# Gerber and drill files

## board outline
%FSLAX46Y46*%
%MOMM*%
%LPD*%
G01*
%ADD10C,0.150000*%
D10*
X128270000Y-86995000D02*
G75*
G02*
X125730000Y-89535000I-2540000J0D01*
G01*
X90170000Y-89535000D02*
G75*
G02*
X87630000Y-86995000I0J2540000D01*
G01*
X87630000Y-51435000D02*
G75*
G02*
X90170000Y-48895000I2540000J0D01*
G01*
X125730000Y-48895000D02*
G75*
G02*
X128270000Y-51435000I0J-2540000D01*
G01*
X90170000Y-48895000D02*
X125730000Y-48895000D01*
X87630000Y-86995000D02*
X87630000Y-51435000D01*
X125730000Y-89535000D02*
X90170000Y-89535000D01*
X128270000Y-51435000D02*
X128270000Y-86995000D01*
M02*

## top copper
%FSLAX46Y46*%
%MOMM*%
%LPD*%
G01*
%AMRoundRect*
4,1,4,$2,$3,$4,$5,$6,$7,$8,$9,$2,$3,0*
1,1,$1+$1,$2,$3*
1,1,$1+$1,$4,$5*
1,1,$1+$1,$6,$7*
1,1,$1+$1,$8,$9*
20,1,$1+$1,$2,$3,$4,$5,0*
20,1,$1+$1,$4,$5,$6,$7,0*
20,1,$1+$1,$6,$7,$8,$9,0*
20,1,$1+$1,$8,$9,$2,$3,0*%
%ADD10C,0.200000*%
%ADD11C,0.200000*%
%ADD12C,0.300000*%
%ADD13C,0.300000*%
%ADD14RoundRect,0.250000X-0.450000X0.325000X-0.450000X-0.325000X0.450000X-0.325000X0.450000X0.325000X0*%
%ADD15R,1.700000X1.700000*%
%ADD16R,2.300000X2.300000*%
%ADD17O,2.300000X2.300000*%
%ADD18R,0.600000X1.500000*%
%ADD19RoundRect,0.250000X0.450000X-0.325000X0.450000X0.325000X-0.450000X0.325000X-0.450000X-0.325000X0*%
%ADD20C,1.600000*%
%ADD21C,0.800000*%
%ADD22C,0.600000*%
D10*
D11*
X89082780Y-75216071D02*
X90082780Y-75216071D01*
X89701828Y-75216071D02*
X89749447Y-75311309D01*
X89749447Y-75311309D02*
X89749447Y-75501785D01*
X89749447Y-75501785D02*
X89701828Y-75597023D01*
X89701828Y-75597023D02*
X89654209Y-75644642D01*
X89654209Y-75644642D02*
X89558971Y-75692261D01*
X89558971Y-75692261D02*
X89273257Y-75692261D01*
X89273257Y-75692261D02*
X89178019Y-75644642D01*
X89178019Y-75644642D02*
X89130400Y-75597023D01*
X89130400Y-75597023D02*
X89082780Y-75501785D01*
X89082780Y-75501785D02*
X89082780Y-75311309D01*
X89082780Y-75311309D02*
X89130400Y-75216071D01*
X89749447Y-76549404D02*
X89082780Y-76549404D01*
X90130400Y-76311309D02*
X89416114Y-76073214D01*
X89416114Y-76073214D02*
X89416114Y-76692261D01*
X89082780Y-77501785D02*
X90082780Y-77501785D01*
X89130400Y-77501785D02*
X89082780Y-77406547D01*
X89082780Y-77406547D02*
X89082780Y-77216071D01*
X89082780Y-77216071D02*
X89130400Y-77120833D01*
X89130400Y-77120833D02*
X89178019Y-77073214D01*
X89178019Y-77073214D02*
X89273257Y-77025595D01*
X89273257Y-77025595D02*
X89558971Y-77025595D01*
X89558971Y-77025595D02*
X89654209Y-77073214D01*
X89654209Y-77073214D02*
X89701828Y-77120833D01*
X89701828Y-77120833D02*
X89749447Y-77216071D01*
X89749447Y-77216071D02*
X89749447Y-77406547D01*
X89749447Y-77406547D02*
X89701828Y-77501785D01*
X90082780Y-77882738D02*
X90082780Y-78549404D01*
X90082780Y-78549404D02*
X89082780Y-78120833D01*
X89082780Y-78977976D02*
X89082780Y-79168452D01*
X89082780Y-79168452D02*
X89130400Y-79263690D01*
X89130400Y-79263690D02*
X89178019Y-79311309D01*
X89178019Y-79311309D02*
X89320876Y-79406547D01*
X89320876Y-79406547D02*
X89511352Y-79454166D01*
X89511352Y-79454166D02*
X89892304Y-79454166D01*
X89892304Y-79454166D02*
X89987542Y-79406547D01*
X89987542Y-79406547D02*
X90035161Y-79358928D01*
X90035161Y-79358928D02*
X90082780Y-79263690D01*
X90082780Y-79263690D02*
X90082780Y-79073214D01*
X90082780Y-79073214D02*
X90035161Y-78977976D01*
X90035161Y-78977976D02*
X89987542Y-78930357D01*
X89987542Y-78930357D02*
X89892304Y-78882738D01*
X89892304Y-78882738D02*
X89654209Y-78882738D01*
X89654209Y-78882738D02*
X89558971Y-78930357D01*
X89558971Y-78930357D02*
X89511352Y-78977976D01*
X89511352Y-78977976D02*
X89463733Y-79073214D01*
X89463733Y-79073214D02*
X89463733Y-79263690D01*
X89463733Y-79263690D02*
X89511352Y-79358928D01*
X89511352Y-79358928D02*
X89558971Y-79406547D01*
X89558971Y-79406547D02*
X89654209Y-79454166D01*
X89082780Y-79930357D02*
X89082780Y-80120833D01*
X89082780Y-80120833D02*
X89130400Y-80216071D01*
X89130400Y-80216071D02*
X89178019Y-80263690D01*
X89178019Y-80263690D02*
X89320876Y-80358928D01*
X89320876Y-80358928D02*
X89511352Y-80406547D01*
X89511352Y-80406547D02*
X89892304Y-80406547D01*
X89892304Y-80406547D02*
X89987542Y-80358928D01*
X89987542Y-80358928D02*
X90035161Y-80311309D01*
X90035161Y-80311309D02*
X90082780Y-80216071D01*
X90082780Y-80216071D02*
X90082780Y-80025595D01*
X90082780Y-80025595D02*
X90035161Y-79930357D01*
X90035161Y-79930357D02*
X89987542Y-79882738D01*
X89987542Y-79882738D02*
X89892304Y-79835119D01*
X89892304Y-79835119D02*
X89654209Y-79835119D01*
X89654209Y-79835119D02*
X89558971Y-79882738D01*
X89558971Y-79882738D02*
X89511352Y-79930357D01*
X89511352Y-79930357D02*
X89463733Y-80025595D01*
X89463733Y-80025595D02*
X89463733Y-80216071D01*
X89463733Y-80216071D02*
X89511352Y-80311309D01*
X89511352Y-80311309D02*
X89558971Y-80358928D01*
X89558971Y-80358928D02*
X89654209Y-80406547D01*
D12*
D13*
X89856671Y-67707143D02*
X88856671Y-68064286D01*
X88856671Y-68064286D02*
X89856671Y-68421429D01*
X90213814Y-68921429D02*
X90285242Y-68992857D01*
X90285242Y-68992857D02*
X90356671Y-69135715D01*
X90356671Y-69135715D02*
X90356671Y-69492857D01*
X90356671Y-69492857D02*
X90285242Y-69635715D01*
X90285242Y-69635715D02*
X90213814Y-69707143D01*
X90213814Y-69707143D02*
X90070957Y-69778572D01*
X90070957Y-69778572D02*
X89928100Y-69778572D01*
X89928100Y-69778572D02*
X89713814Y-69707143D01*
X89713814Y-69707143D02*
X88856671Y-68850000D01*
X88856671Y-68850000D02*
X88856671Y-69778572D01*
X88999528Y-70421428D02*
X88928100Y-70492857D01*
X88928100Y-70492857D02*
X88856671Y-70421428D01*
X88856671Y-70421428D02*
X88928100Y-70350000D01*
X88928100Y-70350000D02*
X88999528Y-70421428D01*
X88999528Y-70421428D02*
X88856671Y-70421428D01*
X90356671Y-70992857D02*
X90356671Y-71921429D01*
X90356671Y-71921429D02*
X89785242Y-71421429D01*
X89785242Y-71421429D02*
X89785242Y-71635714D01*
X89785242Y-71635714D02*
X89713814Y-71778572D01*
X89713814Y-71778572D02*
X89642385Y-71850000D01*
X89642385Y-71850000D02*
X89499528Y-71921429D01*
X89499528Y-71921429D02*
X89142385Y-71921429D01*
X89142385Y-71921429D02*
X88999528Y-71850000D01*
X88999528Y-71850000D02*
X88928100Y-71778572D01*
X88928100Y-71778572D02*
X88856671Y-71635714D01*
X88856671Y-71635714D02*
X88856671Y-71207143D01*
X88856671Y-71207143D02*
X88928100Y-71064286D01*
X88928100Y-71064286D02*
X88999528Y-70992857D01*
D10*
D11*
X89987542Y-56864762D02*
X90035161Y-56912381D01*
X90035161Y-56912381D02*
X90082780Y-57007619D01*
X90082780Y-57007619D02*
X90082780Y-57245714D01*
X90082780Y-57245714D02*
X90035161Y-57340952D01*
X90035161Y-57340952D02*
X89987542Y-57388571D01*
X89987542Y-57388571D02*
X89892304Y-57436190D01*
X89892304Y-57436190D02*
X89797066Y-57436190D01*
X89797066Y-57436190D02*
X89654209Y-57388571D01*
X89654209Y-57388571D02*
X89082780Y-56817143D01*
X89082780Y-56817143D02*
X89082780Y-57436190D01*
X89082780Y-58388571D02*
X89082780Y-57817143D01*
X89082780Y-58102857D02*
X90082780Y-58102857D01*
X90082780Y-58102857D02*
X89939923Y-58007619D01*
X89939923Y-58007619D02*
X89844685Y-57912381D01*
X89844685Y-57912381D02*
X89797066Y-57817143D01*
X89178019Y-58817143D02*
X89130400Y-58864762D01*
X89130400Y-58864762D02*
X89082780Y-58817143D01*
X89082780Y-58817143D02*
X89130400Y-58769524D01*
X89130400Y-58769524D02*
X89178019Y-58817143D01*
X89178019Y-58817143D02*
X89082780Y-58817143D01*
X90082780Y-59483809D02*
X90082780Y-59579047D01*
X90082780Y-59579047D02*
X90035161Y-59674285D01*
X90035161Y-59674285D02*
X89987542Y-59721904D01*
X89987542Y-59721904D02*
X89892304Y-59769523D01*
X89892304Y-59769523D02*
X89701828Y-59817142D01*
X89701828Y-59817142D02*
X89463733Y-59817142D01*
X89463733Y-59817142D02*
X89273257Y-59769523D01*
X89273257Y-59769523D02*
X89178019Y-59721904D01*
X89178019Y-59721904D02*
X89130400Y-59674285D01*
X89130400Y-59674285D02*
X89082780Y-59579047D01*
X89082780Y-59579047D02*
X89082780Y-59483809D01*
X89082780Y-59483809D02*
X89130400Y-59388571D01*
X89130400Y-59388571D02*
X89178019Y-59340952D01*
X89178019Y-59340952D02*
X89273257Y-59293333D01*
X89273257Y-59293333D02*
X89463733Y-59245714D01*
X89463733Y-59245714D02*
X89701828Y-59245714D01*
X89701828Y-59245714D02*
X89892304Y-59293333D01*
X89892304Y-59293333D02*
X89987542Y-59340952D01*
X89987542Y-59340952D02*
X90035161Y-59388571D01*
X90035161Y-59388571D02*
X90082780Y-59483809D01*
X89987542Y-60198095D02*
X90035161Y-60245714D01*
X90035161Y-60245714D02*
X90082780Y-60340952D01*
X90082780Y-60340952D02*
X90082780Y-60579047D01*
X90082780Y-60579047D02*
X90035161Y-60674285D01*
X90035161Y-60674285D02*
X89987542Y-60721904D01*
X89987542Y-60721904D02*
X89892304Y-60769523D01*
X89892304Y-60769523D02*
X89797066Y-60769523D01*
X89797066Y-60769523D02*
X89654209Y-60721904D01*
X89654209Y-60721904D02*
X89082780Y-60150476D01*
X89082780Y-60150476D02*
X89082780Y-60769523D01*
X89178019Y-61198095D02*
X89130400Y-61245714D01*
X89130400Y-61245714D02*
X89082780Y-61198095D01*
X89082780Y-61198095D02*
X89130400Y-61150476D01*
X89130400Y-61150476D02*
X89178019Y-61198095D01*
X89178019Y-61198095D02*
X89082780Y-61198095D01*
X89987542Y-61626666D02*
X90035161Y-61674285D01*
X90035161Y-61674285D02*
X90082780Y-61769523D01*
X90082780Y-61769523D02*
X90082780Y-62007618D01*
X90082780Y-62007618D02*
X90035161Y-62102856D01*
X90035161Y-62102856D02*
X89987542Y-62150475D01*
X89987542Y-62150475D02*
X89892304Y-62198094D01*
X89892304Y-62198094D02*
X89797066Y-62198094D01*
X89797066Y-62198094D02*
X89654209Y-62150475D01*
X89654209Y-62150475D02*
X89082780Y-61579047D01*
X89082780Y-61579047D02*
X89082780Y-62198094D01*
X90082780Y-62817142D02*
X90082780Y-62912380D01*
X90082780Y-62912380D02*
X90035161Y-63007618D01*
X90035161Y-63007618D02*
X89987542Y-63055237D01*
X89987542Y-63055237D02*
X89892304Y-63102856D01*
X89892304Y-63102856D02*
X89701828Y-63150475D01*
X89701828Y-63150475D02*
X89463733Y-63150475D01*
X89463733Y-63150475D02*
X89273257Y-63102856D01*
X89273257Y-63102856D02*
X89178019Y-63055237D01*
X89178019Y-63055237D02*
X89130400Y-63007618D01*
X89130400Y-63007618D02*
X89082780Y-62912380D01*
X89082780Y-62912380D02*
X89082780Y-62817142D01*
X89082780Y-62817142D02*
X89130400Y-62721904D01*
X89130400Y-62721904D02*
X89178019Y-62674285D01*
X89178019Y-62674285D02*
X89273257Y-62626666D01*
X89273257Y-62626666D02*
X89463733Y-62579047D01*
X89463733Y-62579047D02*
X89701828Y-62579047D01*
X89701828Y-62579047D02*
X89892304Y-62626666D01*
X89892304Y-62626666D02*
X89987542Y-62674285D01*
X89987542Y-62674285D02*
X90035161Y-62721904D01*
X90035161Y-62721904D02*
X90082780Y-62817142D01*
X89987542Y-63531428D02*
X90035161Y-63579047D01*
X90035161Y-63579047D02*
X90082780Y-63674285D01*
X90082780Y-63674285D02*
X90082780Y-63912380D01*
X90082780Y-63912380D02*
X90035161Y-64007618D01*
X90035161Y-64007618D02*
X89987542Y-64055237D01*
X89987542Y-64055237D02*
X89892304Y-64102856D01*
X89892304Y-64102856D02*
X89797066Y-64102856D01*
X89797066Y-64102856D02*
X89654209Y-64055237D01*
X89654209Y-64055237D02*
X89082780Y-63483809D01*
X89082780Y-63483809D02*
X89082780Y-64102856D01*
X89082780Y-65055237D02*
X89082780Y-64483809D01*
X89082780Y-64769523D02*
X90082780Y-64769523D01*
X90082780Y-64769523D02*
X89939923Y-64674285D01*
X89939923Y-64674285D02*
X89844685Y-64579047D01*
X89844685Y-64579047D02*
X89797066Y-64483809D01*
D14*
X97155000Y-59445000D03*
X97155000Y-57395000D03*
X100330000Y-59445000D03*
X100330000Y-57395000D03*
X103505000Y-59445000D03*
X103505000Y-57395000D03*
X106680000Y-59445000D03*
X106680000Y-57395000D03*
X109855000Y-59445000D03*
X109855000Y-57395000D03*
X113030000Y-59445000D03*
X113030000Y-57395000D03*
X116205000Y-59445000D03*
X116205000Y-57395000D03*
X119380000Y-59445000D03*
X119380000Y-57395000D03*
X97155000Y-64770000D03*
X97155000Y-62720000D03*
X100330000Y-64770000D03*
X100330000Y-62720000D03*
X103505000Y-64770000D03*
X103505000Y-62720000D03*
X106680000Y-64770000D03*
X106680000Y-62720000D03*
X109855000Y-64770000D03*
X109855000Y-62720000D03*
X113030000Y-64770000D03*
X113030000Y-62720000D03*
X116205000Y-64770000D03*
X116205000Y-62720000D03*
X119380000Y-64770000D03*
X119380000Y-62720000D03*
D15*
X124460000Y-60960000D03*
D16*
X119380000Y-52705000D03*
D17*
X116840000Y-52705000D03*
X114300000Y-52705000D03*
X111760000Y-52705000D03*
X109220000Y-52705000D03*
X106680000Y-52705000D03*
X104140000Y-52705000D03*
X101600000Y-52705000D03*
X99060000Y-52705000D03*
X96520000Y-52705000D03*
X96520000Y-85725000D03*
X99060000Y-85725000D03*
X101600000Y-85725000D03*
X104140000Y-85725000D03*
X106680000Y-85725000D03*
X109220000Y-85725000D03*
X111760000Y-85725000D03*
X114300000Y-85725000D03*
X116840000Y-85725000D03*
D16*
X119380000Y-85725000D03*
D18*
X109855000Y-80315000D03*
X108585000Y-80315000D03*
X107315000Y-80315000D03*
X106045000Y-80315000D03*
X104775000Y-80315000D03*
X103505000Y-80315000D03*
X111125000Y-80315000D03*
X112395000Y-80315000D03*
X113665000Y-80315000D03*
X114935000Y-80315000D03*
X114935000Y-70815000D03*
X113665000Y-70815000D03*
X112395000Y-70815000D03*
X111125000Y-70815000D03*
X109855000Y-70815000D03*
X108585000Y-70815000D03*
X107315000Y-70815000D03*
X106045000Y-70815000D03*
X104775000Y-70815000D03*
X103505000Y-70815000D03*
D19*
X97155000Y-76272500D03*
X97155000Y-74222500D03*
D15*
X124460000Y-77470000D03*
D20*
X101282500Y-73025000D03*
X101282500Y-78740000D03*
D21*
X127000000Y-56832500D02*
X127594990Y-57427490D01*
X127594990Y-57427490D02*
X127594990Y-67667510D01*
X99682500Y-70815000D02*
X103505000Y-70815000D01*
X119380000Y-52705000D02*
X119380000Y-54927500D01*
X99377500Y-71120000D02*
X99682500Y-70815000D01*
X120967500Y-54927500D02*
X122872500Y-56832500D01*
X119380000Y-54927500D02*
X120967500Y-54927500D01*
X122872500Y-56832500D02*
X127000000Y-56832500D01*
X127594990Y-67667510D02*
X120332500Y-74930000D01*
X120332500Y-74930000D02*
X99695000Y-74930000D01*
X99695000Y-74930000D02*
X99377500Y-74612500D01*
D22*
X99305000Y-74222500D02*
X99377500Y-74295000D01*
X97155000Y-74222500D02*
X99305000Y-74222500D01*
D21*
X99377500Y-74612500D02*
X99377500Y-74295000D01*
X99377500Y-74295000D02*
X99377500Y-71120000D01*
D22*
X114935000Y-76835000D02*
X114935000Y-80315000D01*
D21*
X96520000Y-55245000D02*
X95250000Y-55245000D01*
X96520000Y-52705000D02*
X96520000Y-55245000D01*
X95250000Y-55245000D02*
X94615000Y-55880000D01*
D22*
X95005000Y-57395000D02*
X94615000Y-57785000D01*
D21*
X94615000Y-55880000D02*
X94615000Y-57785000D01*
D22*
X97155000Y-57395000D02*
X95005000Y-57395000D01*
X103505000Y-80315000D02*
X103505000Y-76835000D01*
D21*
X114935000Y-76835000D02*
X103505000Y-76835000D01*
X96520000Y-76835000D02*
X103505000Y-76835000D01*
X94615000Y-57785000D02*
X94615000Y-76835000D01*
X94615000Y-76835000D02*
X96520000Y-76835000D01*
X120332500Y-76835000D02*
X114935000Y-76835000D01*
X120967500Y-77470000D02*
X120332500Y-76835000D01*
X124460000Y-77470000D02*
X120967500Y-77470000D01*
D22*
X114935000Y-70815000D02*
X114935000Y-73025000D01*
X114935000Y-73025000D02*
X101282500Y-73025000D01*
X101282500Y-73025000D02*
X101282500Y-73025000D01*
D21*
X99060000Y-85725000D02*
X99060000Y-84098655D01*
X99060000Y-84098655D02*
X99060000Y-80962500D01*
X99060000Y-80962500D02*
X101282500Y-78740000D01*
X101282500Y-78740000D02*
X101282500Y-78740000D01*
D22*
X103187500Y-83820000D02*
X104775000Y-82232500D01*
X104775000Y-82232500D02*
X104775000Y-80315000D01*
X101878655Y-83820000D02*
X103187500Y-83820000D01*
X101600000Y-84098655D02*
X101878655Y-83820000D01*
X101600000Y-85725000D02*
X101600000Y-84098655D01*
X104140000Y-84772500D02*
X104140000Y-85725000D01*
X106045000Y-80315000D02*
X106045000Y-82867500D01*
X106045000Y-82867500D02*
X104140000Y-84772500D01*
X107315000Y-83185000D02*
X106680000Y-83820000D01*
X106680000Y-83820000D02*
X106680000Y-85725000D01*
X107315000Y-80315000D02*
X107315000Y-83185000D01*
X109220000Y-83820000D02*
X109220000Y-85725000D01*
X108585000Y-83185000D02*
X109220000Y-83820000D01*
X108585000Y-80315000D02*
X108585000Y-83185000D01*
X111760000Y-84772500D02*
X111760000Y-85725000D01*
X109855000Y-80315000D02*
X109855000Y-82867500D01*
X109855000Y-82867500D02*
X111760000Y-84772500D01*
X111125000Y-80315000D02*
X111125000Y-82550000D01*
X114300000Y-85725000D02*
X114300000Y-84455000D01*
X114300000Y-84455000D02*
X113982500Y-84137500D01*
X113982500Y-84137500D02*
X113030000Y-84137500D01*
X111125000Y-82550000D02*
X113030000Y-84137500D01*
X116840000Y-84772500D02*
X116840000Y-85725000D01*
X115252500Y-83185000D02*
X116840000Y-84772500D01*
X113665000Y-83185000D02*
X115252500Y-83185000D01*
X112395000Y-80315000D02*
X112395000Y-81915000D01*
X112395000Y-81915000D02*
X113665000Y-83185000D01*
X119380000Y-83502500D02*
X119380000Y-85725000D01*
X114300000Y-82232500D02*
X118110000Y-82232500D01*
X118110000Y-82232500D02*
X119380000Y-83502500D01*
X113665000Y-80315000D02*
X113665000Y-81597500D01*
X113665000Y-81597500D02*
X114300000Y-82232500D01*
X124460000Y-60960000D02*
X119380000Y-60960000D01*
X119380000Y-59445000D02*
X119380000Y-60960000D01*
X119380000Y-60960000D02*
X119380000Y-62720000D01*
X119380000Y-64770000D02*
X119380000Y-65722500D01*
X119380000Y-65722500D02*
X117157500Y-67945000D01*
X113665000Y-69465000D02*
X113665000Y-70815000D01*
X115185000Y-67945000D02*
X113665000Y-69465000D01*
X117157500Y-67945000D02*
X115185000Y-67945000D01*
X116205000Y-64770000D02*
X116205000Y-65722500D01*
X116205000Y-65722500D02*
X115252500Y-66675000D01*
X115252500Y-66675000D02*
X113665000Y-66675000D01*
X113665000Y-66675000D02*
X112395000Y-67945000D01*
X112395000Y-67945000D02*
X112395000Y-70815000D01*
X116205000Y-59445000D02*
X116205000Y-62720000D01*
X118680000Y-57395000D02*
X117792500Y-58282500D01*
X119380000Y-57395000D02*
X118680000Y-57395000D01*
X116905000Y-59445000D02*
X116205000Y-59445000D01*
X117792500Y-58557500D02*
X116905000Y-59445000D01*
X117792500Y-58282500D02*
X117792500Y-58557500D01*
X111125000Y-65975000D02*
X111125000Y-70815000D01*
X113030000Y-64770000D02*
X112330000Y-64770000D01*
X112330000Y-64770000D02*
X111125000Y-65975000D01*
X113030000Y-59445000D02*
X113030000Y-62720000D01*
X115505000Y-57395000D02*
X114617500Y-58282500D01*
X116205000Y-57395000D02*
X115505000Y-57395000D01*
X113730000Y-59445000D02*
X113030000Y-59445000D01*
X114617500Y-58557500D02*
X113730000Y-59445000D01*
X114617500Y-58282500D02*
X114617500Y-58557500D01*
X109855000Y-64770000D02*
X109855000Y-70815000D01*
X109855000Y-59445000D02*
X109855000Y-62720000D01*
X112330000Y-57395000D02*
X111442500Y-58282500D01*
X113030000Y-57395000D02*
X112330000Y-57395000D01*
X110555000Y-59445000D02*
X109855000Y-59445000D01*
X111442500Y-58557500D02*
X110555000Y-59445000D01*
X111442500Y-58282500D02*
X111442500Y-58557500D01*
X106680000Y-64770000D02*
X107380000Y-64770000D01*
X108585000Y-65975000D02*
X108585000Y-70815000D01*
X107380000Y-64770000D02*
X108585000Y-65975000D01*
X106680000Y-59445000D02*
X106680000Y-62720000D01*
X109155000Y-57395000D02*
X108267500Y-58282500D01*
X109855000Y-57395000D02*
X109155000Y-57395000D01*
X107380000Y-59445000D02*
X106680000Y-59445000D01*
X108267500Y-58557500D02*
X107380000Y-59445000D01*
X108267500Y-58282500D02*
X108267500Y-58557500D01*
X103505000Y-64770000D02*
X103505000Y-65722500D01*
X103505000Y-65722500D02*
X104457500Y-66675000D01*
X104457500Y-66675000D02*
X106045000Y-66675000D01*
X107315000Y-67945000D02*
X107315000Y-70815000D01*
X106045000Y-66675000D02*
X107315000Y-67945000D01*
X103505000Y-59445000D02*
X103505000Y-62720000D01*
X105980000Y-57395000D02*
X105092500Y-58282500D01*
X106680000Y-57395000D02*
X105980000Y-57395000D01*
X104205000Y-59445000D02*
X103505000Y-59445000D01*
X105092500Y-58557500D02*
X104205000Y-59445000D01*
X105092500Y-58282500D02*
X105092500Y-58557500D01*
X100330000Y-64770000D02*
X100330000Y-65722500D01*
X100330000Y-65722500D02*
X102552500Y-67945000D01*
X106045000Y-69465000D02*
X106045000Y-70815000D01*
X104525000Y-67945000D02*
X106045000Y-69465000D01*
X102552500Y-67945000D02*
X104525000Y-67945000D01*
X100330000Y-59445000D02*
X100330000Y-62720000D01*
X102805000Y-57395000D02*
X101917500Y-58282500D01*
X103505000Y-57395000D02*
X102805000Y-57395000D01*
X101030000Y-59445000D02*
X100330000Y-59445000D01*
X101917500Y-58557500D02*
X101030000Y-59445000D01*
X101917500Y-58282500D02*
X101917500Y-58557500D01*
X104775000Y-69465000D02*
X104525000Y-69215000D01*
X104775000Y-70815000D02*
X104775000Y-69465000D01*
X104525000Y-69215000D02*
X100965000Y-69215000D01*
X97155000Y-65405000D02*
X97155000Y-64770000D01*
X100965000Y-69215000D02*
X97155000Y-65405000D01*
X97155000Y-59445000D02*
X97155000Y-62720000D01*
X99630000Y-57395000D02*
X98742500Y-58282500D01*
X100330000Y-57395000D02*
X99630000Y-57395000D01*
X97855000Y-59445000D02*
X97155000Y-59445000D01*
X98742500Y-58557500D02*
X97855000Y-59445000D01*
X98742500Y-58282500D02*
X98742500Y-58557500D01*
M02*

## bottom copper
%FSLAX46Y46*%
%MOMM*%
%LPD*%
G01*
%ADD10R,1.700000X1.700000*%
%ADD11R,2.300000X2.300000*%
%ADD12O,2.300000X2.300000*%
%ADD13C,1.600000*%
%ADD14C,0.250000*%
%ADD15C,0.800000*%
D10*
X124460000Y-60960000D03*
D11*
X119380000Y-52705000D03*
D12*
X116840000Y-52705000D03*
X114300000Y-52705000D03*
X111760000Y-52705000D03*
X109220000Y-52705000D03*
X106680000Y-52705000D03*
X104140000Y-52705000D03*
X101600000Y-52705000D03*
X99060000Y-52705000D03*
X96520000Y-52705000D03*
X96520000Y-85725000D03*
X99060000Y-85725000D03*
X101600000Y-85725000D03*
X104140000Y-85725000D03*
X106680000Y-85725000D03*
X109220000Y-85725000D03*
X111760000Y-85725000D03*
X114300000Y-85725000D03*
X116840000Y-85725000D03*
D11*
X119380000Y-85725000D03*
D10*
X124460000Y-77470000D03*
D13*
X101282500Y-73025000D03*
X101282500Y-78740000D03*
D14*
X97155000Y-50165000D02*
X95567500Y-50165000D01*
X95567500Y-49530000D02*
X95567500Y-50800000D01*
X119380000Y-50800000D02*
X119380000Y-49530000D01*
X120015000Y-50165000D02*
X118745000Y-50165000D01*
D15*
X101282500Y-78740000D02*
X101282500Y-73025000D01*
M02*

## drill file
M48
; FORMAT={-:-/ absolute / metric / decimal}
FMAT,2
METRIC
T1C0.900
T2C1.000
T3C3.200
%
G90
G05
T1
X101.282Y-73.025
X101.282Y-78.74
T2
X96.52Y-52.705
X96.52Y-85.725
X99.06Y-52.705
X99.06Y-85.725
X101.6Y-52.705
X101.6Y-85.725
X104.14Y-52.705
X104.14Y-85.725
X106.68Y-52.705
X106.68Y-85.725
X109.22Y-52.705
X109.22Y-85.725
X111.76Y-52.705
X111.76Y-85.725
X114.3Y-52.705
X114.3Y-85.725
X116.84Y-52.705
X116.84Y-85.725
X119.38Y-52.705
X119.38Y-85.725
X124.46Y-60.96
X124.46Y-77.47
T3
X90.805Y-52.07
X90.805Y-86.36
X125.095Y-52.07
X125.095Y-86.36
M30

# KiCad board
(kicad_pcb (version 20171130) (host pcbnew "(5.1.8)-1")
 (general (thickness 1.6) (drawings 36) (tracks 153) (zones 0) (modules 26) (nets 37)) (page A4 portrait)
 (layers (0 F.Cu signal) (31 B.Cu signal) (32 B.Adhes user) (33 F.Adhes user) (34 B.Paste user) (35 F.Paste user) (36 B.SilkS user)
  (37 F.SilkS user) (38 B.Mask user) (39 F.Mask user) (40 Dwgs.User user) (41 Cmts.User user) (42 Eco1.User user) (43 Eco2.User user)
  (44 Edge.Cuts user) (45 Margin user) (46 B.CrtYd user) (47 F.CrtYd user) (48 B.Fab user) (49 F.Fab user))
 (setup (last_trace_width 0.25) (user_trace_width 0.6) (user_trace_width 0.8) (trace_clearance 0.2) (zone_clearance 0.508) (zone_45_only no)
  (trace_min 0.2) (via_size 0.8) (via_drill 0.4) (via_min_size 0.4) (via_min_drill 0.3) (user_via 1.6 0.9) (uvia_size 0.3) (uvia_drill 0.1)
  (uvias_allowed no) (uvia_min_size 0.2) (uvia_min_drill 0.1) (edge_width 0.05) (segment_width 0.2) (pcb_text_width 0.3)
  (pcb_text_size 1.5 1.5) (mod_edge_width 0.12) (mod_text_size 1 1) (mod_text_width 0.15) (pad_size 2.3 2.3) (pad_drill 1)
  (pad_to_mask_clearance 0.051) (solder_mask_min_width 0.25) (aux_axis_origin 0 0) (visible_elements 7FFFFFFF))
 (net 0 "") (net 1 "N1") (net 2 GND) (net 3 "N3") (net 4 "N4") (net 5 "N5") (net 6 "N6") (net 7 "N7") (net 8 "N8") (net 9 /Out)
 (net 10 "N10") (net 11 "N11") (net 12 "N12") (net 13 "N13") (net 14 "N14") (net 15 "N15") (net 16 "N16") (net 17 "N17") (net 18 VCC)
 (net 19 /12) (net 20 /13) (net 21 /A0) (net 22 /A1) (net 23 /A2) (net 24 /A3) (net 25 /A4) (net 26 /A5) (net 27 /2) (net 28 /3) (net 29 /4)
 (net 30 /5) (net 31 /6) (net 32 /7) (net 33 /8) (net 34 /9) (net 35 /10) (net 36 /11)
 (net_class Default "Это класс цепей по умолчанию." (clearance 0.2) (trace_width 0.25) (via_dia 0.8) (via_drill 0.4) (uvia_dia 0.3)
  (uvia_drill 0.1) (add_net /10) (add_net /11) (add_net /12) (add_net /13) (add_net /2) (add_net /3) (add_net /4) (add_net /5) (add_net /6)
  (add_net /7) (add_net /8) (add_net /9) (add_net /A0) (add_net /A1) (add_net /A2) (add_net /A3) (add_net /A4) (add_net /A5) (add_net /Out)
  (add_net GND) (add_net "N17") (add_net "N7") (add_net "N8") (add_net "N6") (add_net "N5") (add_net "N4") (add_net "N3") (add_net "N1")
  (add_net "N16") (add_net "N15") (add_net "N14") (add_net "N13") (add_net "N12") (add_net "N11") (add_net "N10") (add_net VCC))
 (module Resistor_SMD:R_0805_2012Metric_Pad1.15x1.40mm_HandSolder (layer F.Cu) (at 97.155 58.42 270)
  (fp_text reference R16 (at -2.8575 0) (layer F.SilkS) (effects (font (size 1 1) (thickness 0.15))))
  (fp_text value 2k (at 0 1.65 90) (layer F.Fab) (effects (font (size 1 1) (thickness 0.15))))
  (pad 2 smd roundrect (at 1.025 0 270) (size 1.15 1.4) (layers F.Cu F.Paste F.Mask) (roundrect_rratio 0.217391) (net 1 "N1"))
  (pad 1 smd roundrect (at -1.025 0 270) (size 1.15 1.4) (layers F.Cu F.Paste F.Mask) (roundrect_rratio 0.217391) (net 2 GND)))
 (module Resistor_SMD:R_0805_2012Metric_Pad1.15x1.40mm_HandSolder (layer F.Cu) (at 100.33 58.42 270)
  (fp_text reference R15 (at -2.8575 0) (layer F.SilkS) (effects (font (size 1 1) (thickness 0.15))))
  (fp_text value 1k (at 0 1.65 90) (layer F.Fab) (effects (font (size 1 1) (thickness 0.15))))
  (pad 2 smd roundrect (at 1.025 0 270) (size 1.15 1.4) (layers F.Cu F.Paste F.Mask) (roundrect_rratio 0.217391) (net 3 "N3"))
  (pad 1 smd roundrect (at -1.025 0 270) (size 1.15 1.4) (layers F.Cu F.Paste F.Mask) (roundrect_rratio 0.217391) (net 1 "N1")))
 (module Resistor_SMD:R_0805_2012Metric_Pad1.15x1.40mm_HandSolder (layer F.Cu) (at 103.505 58.42 270)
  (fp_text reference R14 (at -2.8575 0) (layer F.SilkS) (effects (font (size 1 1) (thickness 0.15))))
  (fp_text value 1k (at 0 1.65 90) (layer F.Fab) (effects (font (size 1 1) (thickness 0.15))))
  (pad 2 smd roundrect (at 1.025 0 270) (size 1.15 1.4) (layers F.Cu F.Paste F.Mask) (roundrect_rratio 0.217391) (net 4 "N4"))
  (pad 1 smd roundrect (at -1.025 0 270) (size 1.15 1.4) (layers F.Cu F.Paste F.Mask) (roundrect_rratio 0.217391) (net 3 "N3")))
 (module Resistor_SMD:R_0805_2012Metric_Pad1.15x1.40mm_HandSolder (layer F.Cu) (at 106.68 58.42 270)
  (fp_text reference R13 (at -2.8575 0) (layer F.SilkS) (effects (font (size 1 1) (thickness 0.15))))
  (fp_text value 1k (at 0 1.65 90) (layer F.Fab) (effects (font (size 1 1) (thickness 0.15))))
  (pad 2 smd roundrect (at 1.025 0 270) (size 1.15 1.4) (layers F.Cu F.Paste F.Mask) (roundrect_rratio 0.217391) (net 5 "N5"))
  (pad 1 smd roundrect (at -1.025 0 270) (size 1.15 1.4) (layers F.Cu F.Paste F.Mask) (roundrect_rratio 0.217391) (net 4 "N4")))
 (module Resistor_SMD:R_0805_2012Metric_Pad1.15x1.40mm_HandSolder (layer F.Cu) (at 109.855 58.42 270)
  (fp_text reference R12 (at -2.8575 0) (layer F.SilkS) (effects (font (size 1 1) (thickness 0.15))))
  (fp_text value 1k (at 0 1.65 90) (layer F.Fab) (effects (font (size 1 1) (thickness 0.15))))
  (pad 2 smd roundrect (at 1.025 0 270) (size 1.15 1.4) (layers F.Cu F.Paste F.Mask) (roundrect_rratio 0.217391) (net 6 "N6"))
  (pad 1 smd roundrect (at -1.025 0 270) (size 1.15 1.4) (layers F.Cu F.Paste F.Mask) (roundrect_rratio 0.217391) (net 5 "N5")))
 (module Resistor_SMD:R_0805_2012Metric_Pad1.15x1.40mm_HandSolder (layer F.Cu) (at 113.03 58.42 270)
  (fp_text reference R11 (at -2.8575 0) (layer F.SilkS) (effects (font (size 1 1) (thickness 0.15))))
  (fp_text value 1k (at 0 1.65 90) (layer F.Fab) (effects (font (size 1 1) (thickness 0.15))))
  (pad 2 smd roundrect (at 1.025 0 270) (size 1.15 1.4) (layers F.Cu F.Paste F.Mask) (roundrect_rratio 0.217391) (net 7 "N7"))
  (pad 1 smd roundrect (at -1.025 0 270) (size 1.15 1.4) (layers F.Cu F.Paste F.Mask) (roundrect_rratio 0.217391) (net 6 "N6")))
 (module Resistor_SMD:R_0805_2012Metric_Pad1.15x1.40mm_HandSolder (layer F.Cu) (at 116.205 58.42 270)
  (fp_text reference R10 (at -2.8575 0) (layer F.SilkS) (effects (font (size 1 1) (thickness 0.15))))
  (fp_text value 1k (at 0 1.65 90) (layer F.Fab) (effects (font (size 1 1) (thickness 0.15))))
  (pad 2 smd roundrect (at 1.025 0 270) (size 1.15 1.4) (layers F.Cu F.Paste F.Mask) (roundrect_rratio 0.217391) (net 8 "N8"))
  (pad 1 smd roundrect (at -1.025 0 270) (size 1.15 1.4) (layers F.Cu F.Paste F.Mask) (roundrect_rratio 0.217391) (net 7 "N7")))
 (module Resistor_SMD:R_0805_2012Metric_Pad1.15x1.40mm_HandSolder (layer F.Cu) (at 119.38 58.42 270)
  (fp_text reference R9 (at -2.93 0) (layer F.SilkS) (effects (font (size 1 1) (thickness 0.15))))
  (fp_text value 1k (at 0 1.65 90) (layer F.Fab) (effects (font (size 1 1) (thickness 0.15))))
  (pad 2 smd roundrect (at 1.025 0 270) (size 1.15 1.4) (layers F.Cu F.Paste F.Mask) (roundrect_rratio 0.217391) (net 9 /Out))
  (pad 1 smd roundrect (at -1.025 0 270) (size 1.15 1.4) (layers F.Cu F.Paste F.Mask) (roundrect_rratio 0.217391) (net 8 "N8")))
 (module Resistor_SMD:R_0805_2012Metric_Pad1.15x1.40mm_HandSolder (layer F.Cu) (at 97.155 63.745 270)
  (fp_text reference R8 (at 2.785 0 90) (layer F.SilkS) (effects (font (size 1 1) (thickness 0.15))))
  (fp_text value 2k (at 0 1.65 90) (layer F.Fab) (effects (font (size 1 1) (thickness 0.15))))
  (pad 2 smd roundrect (at 1.025 0 270) (size 1.15 1.4) (layers F.Cu F.Paste F.Mask) (roundrect_rratio 0.217391) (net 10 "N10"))
  (pad 1 smd roundrect (at -1.025 0 270) (size 1.15 1.4) (layers F.Cu F.Paste F.Mask) (roundrect_rratio 0.217391) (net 1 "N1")))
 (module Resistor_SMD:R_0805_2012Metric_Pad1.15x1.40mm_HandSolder (layer F.Cu) (at 100.33 63.745 270)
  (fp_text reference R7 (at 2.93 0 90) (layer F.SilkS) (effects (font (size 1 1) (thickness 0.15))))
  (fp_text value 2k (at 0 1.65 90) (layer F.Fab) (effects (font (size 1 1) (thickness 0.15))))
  (pad 2 smd roundrect (at 1.025 0 270) (size 1.15 1.4) (layers F.Cu F.Paste F.Mask) (roundrect_rratio 0.217391) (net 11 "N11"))
  (pad 1 smd roundrect (at -1.025 0 270) (size 1.15 1.4) (layers F.Cu F.Paste F.Mask) (roundrect_rratio 0.217391) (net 3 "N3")))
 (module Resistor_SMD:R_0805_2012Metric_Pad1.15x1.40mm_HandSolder (layer F.Cu) (at 103.505 63.745 270)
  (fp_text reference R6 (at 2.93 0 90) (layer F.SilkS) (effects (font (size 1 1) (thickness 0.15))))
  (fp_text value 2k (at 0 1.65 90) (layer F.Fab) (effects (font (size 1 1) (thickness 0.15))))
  (pad 2 smd roundrect (at 1.025 0 270) (size 1.15 1.4) (layers F.Cu F.Paste F.Mask) (roundrect_rratio 0.217391) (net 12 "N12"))
  (pad 1 smd roundrect (at -1.025 0 270) (size 1.15 1.4) (layers F.Cu F.Paste F.Mask) (roundrect_rratio 0.217391) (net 4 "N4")))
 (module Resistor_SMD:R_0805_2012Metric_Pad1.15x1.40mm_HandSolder (layer F.Cu) (at 106.68 63.745 270)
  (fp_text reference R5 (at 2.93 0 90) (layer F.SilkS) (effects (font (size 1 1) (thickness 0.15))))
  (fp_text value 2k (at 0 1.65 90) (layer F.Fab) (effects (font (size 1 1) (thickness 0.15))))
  (pad 2 smd roundrect (at 1.025 0 270) (size 1.15 1.4) (layers F.Cu F.Paste F.Mask) (roundrect_rratio 0.217391) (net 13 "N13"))
  (pad 1 smd roundrect (at -1.025 0 270) (size 1.15 1.4) (layers F.Cu F.Paste F.Mask) (roundrect_rratio 0.217391) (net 5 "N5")))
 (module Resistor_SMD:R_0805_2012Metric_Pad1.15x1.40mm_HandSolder (layer F.Cu) (at 109.855 63.745 270)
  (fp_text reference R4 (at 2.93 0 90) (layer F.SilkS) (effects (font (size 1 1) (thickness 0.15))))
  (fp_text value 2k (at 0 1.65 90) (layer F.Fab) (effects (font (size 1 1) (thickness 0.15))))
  (pad 2 smd roundrect (at 1.025 0 270) (size 1.15 1.4) (layers F.Cu F.Paste F.Mask) (roundrect_rratio 0.217391) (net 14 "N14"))
  (pad 1 smd roundrect (at -1.025 0 270) (size 1.15 1.4) (layers F.Cu F.Paste F.Mask) (roundrect_rratio 0.217391) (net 6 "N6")))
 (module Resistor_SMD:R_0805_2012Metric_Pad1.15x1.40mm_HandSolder (layer F.Cu) (at 113.03 63.745 270)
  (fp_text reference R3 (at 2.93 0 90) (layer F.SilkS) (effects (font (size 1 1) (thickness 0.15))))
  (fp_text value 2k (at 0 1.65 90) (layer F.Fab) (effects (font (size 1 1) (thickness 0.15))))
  (pad 2 smd roundrect (at 1.025 0 270) (size 1.15 1.4) (layers F.Cu F.Paste F.Mask) (roundrect_rratio 0.217391) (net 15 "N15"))
  (pad 1 smd roundrect (at -1.025 0 270) (size 1.15 1.4) (layers F.Cu F.Paste F.Mask) (roundrect_rratio 0.217391) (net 7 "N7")))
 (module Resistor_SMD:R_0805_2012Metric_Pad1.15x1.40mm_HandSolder (layer F.Cu) (at 116.205 63.745 270)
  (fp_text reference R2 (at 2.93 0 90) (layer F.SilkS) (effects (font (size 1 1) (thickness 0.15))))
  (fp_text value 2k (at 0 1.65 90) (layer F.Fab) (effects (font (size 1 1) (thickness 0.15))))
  (pad 2 smd roundrect (at 1.025 0 270) (size 1.15 1.4) (layers F.Cu F.Paste F.Mask) (roundrect_rratio 0.217391) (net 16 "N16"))
  (pad 1 smd roundrect (at -1.025 0 270) (size 1.15 1.4) (layers F.Cu F.Paste F.Mask) (roundrect_rratio 0.217391) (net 8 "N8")))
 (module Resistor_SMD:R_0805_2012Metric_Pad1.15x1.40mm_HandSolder (layer F.Cu) (at 119.38 63.745 270)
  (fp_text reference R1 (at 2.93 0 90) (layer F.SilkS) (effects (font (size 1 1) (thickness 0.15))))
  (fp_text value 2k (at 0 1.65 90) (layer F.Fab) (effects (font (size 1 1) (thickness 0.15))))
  (pad 2 smd roundrect (at 1.025 0 270) (size 1.15 1.4) (layers F.Cu F.Paste F.Mask) (roundrect_rratio 0.217391) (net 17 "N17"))
  (pad 1 smd roundrect (at -1.025 0 270) (size 1.15 1.4) (layers F.Cu F.Paste F.Mask) (roundrect_rratio 0.217391) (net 9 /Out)))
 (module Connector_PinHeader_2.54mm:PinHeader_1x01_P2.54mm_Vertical (layer F.Cu) (at 124.46 60.96 270)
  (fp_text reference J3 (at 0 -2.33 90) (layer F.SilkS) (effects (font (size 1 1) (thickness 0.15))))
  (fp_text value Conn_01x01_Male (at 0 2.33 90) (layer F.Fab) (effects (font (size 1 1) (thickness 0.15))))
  (pad 1 thru_hole rect (at 0 0 270) (size 1.7 1.7) (drill 1) (layers *.Cu *.Mask) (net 9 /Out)))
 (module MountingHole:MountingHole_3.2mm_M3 (layer F.Cu) (at 125.095 52.07 270)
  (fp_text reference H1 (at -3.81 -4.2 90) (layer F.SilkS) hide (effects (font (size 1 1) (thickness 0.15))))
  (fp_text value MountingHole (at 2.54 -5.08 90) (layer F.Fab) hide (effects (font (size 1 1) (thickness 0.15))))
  (pad 1 np_thru_hole circle (at 0 0 270) (size 3.2 3.2) (drill 3.2) (layers *.Cu *.Mask)))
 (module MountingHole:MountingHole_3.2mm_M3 (layer F.Cu) (at 90.805 52.07 270)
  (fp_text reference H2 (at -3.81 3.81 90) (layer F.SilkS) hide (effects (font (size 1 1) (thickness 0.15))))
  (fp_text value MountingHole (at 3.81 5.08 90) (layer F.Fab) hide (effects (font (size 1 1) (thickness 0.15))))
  (pad 1 np_thru_hole circle (at 0 0 270) (size 3.2 3.2) (drill 3.2) (layers *.Cu *.Mask)))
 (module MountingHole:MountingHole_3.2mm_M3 (layer F.Cu) (at 125.095 86.36 270)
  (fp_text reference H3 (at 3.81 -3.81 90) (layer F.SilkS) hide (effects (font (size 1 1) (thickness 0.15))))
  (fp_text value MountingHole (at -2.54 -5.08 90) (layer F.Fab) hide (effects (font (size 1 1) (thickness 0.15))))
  (pad 1 np_thru_hole circle (at 0 0 270) (size 3.2 3.2) (drill 3.2) (layers *.Cu *.Mask)))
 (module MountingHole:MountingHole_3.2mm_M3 (layer F.Cu) (at 90.805 86.36 270)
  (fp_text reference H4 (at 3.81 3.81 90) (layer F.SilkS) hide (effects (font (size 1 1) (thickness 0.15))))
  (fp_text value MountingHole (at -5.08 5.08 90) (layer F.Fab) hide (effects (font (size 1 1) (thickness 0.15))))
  (pad 1 np_thru_hole circle (at 0 0 270) (size 3.2 3.2) (drill 3.2) (layers *.Cu *.Mask)))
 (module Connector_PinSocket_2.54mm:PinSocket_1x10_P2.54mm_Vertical (layer F.Cu) (at 119.38 52.705 270)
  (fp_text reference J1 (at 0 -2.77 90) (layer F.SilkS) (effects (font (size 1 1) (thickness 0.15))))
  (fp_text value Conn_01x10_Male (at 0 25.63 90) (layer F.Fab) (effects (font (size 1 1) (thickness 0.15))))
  (pad 1 thru_hole rect (at 0 0 270) (size 2.3 2.3) (drill 1) (layers *.Cu *.Mask) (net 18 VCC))
  (pad 2 thru_hole oval (at 0 2.54 270) (size 2.3 2.3) (drill 1) (layers *.Cu *.Mask) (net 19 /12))
  (pad 3 thru_hole oval (at 0 5.08 270) (size 2.3 2.3) (drill 1) (layers *.Cu *.Mask) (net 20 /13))
  (pad 4 thru_hole oval (at 0 7.62 270) (size 2.3 2.3) (drill 1) (layers *.Cu *.Mask) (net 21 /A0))
  (pad 5 thru_hole oval (at 0 10.16 270) (size 2.3 2.3) (drill 1) (layers *.Cu *.Mask) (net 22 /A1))
  (pad 6 thru_hole oval (at 0 12.7 270) (size 2.3 2.3) (drill 1) (layers *.Cu *.Mask) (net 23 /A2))
  (pad 7 thru_hole oval (at 0 15.24 270) (size 2.3 2.3) (drill 1) (layers *.Cu *.Mask) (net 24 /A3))
  (pad 8 thru_hole oval (at 0 17.78 270) (size 2.3 2.3) (drill 1) (layers *.Cu *.Mask) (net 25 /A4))
  (pad 9 thru_hole oval (at 0 20.32 270) (size 2.3 2.3) (drill 1) (layers *.Cu *.Mask) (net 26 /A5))
  (pad 10 thru_hole oval (at 0 22.86 270) (size 2.3 2.3) (drill 1) (layers *.Cu *.Mask) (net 2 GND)))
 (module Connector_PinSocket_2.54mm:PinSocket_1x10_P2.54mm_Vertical (layer F.Cu) (at 119.38 85.725 270)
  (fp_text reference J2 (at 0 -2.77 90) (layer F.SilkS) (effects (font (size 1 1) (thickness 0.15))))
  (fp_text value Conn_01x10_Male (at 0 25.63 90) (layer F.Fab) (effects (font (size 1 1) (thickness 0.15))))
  (pad 10 thru_hole oval (at 0 22.86 270) (size 2.3 2.3) (drill 1) (layers *.Cu *.Mask) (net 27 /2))
  (pad 9 thru_hole oval (at 0 20.32 270) (size 2.3 2.3) (drill 1) (layers *.Cu *.Mask) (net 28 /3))
  (pad 8 thru_hole oval (at 0 17.78 270) (size 2.3 2.3) (drill 1) (layers *.Cu *.Mask) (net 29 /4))
  (pad 7 thru_hole oval (at 0 15.24 270) (size 2.3 2.3) (drill 1) (layers *.Cu *.Mask) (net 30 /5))
  (pad 6 thru_hole oval (at 0 12.7 270) (size 2.3 2.3) (drill 1) (layers *.Cu *.Mask) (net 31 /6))
  (pad 5 thru_hole oval (at 0 10.16 270) (size 2.3 2.3) (drill 1) (layers *.Cu *.Mask) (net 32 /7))
  (pad 4 thru_hole oval (at 0 7.62 270) (size 2.3 2.3) (drill 1) (layers *.Cu *.Mask) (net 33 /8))
  (pad 3 thru_hole oval (at 0 5.08 270) (size 2.3 2.3) (drill 1) (layers *.Cu *.Mask) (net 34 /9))
  (pad 2 thru_hole oval (at 0 2.54 270) (size 2.3 2.3) (drill 1) (layers *.Cu *.Mask) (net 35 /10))
  (pad 1 thru_hole rect (at 0 0 270) (size 2.3 2.3) (drill 1) (layers *.Cu *.Mask) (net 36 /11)))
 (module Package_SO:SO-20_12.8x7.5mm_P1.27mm (layer F.Cu) (at 109.22 75.565 90)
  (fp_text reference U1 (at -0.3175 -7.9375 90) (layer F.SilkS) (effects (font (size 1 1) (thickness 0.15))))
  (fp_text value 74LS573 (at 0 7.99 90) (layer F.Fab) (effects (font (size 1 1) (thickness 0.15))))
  (pad 6 smd rect (at -4.75 0.635 90) (size 1.5 0.6) (layers F.Cu F.Paste F.Mask) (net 33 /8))
  (pad 5 smd rect (at -4.75 -0.635 90) (size 1.5 0.6) (layers F.Cu F.Paste F.Mask) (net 32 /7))
  (pad 4 smd rect (at -4.75 -1.905 90) (size 1.5 0.6) (layers F.Cu F.Paste F.Mask) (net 31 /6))
  (pad 3 smd rect (at -4.75 -3.175 90) (size 1.5 0.6) (layers F.Cu F.Paste F.Mask) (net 30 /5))
  (pad 2 smd rect (at -4.75 -4.445 90) (size 1.5 0.6) (layers F.Cu F.Paste F.Mask) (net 29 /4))
  (pad 1 smd rect (at -4.75 -5.715 90) (size 1.5 0.6) (layers F.Cu F.Paste F.Mask) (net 2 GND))
  (pad 7 smd rect (at -4.75 1.905 90) (size 1.5 0.6) (layers F.Cu F.Paste F.Mask) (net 34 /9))
  (pad 8 smd rect (at -4.75 3.175 90) (size 1.5 0.6) (layers F.Cu F.Paste F.Mask) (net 35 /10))
  (pad 9 smd rect (at -4.75 4.445 90) (size 1.5 0.6) (layers F.Cu F.Paste F.Mask) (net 36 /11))
  (pad 10 smd rect (at -4.75 5.715 90) (size 1.5 0.6) (layers F.Cu F.Paste F.Mask) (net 2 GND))
  (pad 11 smd rect (at 4.75 5.715 90) (size 1.5 0.6) (layers F.Cu F.Paste F.Mask) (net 28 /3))
  (pad 12 smd rect (at 4.75 4.445 90) (size 1.5 0.6) (layers F.Cu F.Paste F.Mask) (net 17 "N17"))
  (pad 13 smd rect (at 4.75 3.175 90) (size 1.5 0.6) (layers F.Cu F.Paste F.Mask) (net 16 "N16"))
  (pad 14 smd rect (at 4.75 1.905 90) (size 1.5 0.6) (layers F.Cu F.Paste F.Mask) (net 15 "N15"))
  (pad 15 smd rect (at 4.75 0.635 90) (size 1.5 0.6) (layers F.Cu F.Paste F.Mask) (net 14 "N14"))
  (pad 16 smd rect (at 4.75 -0.635 90) (size 1.5 0.6) (layers F.Cu F.Paste F.Mask) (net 13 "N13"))
  (pad 17 smd rect (at 4.75 -1.905 90) (size 1.5 0.6) (layers F.Cu F.Paste F.Mask) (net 12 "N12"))
  (pad 18 smd rect (at 4.75 -3.175 90) (size 1.5 0.6) (layers F.Cu F.Paste F.Mask) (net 11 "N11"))
  (pad 19 smd rect (at 4.75 -4.445 90) (size 1.5 0.6) (layers F.Cu F.Paste F.Mask) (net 10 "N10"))
  (pad 20 smd rect (at 4.75 -5.715 90) (size 1.5 0.6) (layers F.Cu F.Paste F.Mask) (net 18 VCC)))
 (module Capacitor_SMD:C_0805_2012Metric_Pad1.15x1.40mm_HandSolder (layer F.Cu) (at 97.155 75.2475 90)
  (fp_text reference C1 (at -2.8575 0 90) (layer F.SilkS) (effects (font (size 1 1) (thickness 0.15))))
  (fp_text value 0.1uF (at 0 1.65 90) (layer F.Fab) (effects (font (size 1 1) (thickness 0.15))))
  (pad 1 smd roundrect (at -1.025 0 90) (size 1.15 1.4) (layers F.Cu F.Paste F.Mask) (roundrect_rratio 0.217391) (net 2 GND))
  (pad 2 smd roundrect (at 1.025 0 90) (size 1.15 1.4) (layers F.Cu F.Paste F.Mask) (roundrect_rratio 0.217391) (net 18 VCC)))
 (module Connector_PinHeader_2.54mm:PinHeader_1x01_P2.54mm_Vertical (layer F.Cu) (at 124.46 77.47 270)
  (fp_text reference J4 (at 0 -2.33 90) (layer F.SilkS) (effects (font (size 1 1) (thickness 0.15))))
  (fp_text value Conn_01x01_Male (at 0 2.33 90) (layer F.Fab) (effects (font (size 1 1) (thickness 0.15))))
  (pad 1 thru_hole rect (at 0 0 270) (size 1.7 1.7) (drill 1) (layers *.Cu *.Mask) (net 2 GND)))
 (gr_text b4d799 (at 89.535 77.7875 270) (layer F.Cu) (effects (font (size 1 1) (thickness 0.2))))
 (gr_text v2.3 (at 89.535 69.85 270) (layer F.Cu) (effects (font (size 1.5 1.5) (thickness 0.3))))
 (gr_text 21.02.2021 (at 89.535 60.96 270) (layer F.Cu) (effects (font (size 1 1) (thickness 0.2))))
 (gr_arc (start 125.73 86.995) (end 125.73 89.535) (angle -90) (layer Edge.Cuts) (width 0.15))
 (gr_arc (start 90.17 86.995) (end 87.63 86.995) (angle -90) (layer Edge.Cuts) (width 0.15))
 (gr_arc (start 90.17 51.435) (end 90.17 48.895) (angle -90) (layer Edge.Cuts) (width 0.15))
 (gr_arc (start 125.73 51.435) (end 128.27 51.435) (angle -90) (layer Edge.Cuts) (width 0.15))
 (gr_line (start 90.17 48.895) (end 125.73 48.895) (layer Edge.Cuts) (width 0.15))
 (gr_line (start 87.63 86.995) (end 87.63 51.435) (layer Edge.Cuts) (width 0.15))
 (gr_line (start 125.73 89.535) (end 90.17 89.535) (layer Edge.Cuts) (width 0.15))
 (gr_line (start 128.27 51.435) (end 128.27 86.995) (layer Edge.Cuts) (width 0.15))
 (segment (start 97.155 50.165) (end 95.5675 50.165) (width 0.25) (layer B.Cu) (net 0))
 (segment (start 95.5675 49.53) (end 95.5675 50.8) (width 0.25) (layer B.Cu) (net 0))
 (segment (start 119.38 50.8) (end 119.38 49.53) (width 0.25) (layer B.Cu) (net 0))
 (segment (start 120.015 50.165) (end 118.745 50.165) (width 0.25) (layer B.Cu) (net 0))
 (segment (start 127 56.8325) (end 127.59499 57.42749) (width 0.8) (layer F.Cu) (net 18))
 (segment (start 127.59499 57.42749) (end 127.59499 67.66751) (width 0.8) (layer F.Cu) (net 18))
 (segment (start 99.6825 70.815) (end 103.505 70.815) (width 0.8) (layer F.Cu) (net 18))
 (segment (start 119.38 52.705) (end 119.38 54.9275) (width 0.8) (layer F.Cu) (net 18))
 (segment (start 99.3775 71.12) (end 99.6825 70.815) (width 0.8) (layer F.Cu) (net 18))
 (segment (start 120.9675 54.9275) (end 122.8725 56.8325) (width 0.8) (layer F.Cu) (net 18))
 (segment (start 119.38 54.9275) (end 120.9675 54.9275) (width 0.8) (layer F.Cu) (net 18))
 (segment (start 122.8725 56.8325) (end 127 56.8325) (width 0.8) (layer F.Cu) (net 18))
 (segment (start 127.59499 67.66751) (end 120.3325 74.93) (width 0.8) (layer F.Cu) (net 18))
 (segment (start 120.3325 74.93) (end 99.695 74.93) (width 0.8) (layer F.Cu) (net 18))
 (segment (start 99.695 74.93) (end 99.3775 74.6125) (width 0.8) (layer F.Cu) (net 18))
 (segment (start 99.305 74.2225) (end 99.3775 74.295) (width 0.6) (layer F.Cu) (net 18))
 (segment (start 97.155 74.2225) (end 99.305 74.2225) (width 0.6) (layer F.Cu) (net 18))
 (segment (start 99.3775 74.6125) (end 99.3775 74.295) (width 0.8) (layer F.Cu) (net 18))
 (segment (start 99.3775 74.295) (end 99.3775 71.12) (width 0.8) (layer F.Cu) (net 18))
 (segment (start 114.935 76.835) (end 114.935 80.315) (width 0.6) (layer F.Cu) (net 2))
 (segment (start 96.52 55.245) (end 95.25 55.245) (width 0.8) (layer F.Cu) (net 2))
 (segment (start 96.52 52.705) (end 96.52 55.245) (width 0.8) (layer F.Cu) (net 2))
 (segment (start 95.25 55.245) (end 94.615 55.88) (width 0.8) (layer F.Cu) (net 2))
 (segment (start 95.005 57.395) (end 94.615 57.785) (width 0.6) (layer F.Cu) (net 2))
 (segment (start 94.615 55.88) (end 94.615 57.785) (width 0.8) (layer F.Cu) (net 2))
 (segment (start 97.155 57.395) (end 95.005 57.395) (width 0.6) (layer F.Cu) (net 2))
 (segment (start 103.505 80.315) (end 103.505 76.835) (width 0.6) (layer F.Cu) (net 2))
 (segment (start 114.935 76.835) (end 103.505 76.835) (width 0.8) (layer F.Cu) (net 2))
 (segment (start 96.52 76.835) (end 103.505 76.835) (width 0.8) (layer F.Cu) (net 2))
 (segment (start 94.615 57.785) (end 94.615 76.835) (width 0.8) (layer F.Cu) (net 2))
 (segment (start 94.615 76.835) (end 96.52 76.835) (width 0.8) (layer F.Cu) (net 2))
 (segment (start 120.3325 76.835) (end 114.935 76.835) (width 0.8) (layer F.Cu) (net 2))
 (segment (start 120.9675 77.47) (end 120.3325 76.835) (width 0.8) (layer F.Cu) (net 2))
 (segment (start 124.46 77.47) (end 120.9675 77.47) (width 0.8) (layer F.Cu) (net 2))
 (segment (start 114.935 70.815) (end 114.935 73.025) (width 0.6) (layer F.Cu) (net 28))
 (segment (start 114.935 73.025) (end 101.2825 73.025) (width 0.6) (layer F.Cu) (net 28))
 (segment (start 101.2825 73.025) (end 101.2825 73.025) (width 0.6) (layer F.Cu) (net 28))
 (via (at 101.2825 73.025) (size 1.6) (drill 0.9) (layers F.Cu B.Cu) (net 28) (status 1000000))
 (segment (start 99.06 85.725) (end 99.06 84.098655) (width 0.8) (layer F.Cu) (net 28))
 (segment (start 99.06 84.098655) (end 99.06 80.9625) (width 0.8) (layer F.Cu) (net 28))
 (segment (start 99.06 80.9625) (end 101.2825 78.74) (width 0.8) (layer F.Cu) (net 28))
 (segment (start 101.2825 78.74) (end 101.2825 78.74) (width 0.8) (layer F.Cu) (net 28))
 (via (at 101.2825 78.74) (size 1.6) (drill 0.9) (layers F.Cu B.Cu) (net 28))
 (segment (start 101.2825 78.74) (end 101.2825 73.025) (width 0.8) (layer B.Cu) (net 28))
 (segment (start 103.1875 83.82) (end 104.775 82.2325) (width 0.6) (layer F.Cu) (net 29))
 (segment (start 104.775 82.2325) (end 104.775 80.315) (width 0.6) (layer F.Cu) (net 29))
 (segment (start 101.878655 83.82) (end 103.1875 83.82) (width 0.6) (layer F.Cu) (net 29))
 (segment (start 101.6 84.098655) (end 101.878655 83.82) (width 0.6) (layer F.Cu) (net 29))
 (segment (start 101.6 85.725) (end 101.6 84.098655) (width 0.6) (layer F.Cu) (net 29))
 (segment (start 104.14 84.7725) (end 104.14 85.725) (width 0.6) (layer F.Cu) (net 30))
 (segment (start 106.045 80.315) (end 106.045 82.8675) (width 0.6) (layer F.Cu) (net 30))
 (segment (start 106.045 82.8675) (end 104.14 84.7725) (width 0.6) (layer F.Cu) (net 30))
 (segment (start 107.315 83.185) (end 106.68 83.82) (width 0.6) (layer F.Cu) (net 31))
 (segment (start 106.68 83.82) (end 106.68 85.725) (width 0.6) (layer F.Cu) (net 31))
 (segment (start 107.315 80.315) (end 107.315 83.185) (width 0.6) (layer F.Cu) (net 31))
 (segment (start 109.22 83.82) (end 109.22 85.725) (width 0.6) (layer F.Cu) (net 32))
 (segment (start 108.585 83.185) (end 109.22 83.82) (width 0.6) (layer F.Cu) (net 32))
 (segment (start 108.585 80.315) (end 108.585 83.185) (width 0.6) (layer F.Cu) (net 32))
 (segment (start 111.76 84.7725) (end 111.76 85.725) (width 0.6) (layer F.Cu) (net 33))
 (segment (start 109.855 80.315) (end 109.855 82.8675) (width 0.6) (layer F.Cu) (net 33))
 (segment (start 109.855 82.8675) (end 111.76 84.7725) (width 0.6) (layer F.Cu) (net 33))
 (segment (start 111.125 80.315) (end 111.125 82.55) (width 0.6) (layer F.Cu) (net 34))
 (segment (start 114.3 85.725) (end 114.3 84.455) (width 0.6) (layer F.Cu) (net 34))
 (segment (start 114.3 84.455) (end 113.9825 84.1375) (width 0.6) (layer F.Cu) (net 34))
 (segment (start 113.9825 84.1375) (end 113.03 84.1375) (width 0.6) (layer F.Cu) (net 34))
 (segment (start 111.125 82.55) (end 113.03 84.1375) (width 0.6) (layer F.Cu) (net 34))
 (segment (start 116.84 84.7725) (end 116.84 85.725) (width 0.6) (layer F.Cu) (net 35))
 (segment (start 115.2525 83.185) (end 116.84 84.7725) (width 0.6) (layer F.Cu) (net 35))
 (segment (start 113.665 83.185) (end 115.2525 83.185) (width 0.6) (layer F.Cu) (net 35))
 (segment (start 112.395 80.315) (end 112.395 81.915) (width 0.6) (layer F.Cu) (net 35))
 (segment (start 112.395 81.915) (end 113.665 83.185) (width 0.6) (layer F.Cu) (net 35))
 (segment (start 119.38 83.5025) (end 119.38 85.725) (width 0.6) (layer F.Cu) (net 36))
 (segment (start 114.3 82.2325) (end 118.11 82.2325) (width 0.6) (layer F.Cu) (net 36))
 (segment (start 118.11 82.2325) (end 119.38 83.5025) (width 0.6) (layer F.Cu) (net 36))
 (segment (start 113.665 80.315) (end 113.665 81.5975) (width 0.6) (layer F.Cu) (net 36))
 (segment (start 113.665 81.5975) (end 114.3 82.2325) (width 0.6) (layer F.Cu) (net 36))
 (segment (start 124.46 60.96) (end 119.38 60.96) (width 0.6) (layer F.Cu) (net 9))
 (segment (start 119.38 59.445) (end 119.38 60.96) (width 0.6) (layer F.Cu) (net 9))
 (segment (start 119.38 60.96) (end 119.38 62.72) (width 0.6) (layer F.Cu) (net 9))
 (segment (start 119.38 64.77) (end 119.38 65.7225) (width 0.6) (layer F.Cu) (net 17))
 (segment (start 119.38 65.7225) (end 117.1575 67.945) (width 0.6) (layer F.Cu) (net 17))
 (segment (start 113.665 69.465) (end 113.665 70.815) (width 0.6) (layer F.Cu) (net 17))
 (segment (start 115.185 67.945) (end 113.665 69.465) (width 0.6) (layer F.Cu) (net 17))
 (segment (start 117.1575 67.945) (end 115.185 67.945) (width 0.6) (layer F.Cu) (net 17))
 (segment (start 116.205 64.77) (end 116.205 65.7225) (width 0.6) (layer F.Cu) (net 16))
 (segment (start 116.205 65.7225) (end 115.2525 66.675) (width 0.6) (layer F.Cu) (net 16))
 (segment (start 115.2525 66.675) (end 113.665 66.675) (width 0.6) (layer F.Cu) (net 16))
 (segment (start 113.665 66.675) (end 112.395 67.945) (width 0.6) (layer F.Cu) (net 16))
 (segment (start 112.395 67.945) (end 112.395 70.815) (width 0.6) (layer F.Cu) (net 16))
 (segment (start 116.205 59.445) (end 116.205 62.72) (width 0.6) (layer F.Cu) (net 8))
 (segment (start 118.68 57.395) (end 117.7925 58.2825) (width 0.6) (layer F.Cu) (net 8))
 (segment (start 119.38 57.395) (end 118.68 57.395) (width 0.6) (layer F.Cu) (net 8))
 (segment (start 116.905 59.445) (end 116.205 59.445) (width 0.6) (layer F.Cu) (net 8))
 (segment (start 117.7925 58.5575) (end 116.905 59.445) (width 0.6) (layer F.Cu) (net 8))
 (segment (start 117.7925 58.2825) (end 117.7925 58.5575) (width 0.6) (layer F.Cu) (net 8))
 (segment (start 111.125 65.975) (end 111.125 70.815) (width 0.6) (layer F.Cu) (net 15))
 (segment (start 113.03 64.77) (end 112.33 64.77) (width 0.6) (layer F.Cu) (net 15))
 (segment (start 112.33 64.77) (end 111.125 65.975) (width 0.6) (layer F.Cu) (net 15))
 (segment (start 113.03 59.445) (end 113.03 62.72) (width 0.6) (layer F.Cu) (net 7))
 (segment (start 115.505 57.395) (end 114.6175 58.2825) (width 0.6) (layer F.Cu) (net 7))
 (segment (start 116.205 57.395) (end 115.505 57.395) (width 0.6) (layer F.Cu) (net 7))
 (segment (start 113.73 59.445) (end 113.03 59.445) (width 0.6) (layer F.Cu) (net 7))
 (segment (start 114.6175 58.5575) (end 113.73 59.445) (width 0.6) (layer F.Cu) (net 7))
 (segment (start 114.6175 58.2825) (end 114.6175 58.5575) (width 0.6) (layer F.Cu) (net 7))
 (segment (start 109.855 64.77) (end 109.855 70.815) (width 0.6) (layer F.Cu) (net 14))
 (segment (start 109.855 59.445) (end 109.855 62.72) (width 0.6) (layer F.Cu) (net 6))
 (segment (start 112.33 57.395) (end 111.4425 58.2825) (width 0.6) (layer F.Cu) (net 6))
 (segment (start 113.03 57.395) (end 112.33 57.395) (width 0.6) (layer F.Cu) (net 6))
 (segment (start 110.555 59.445) (end 109.855 59.445) (width 0.6) (layer F.Cu) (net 6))
 (segment (start 111.4425 58.5575) (end 110.555 59.445) (width 0.6) (layer F.Cu) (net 6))
 (segment (start 111.4425 58.2825) (end 111.4425 58.5575) (width 0.6) (layer F.Cu) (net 6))
 (segment (start 106.68 64.77) (end 107.38 64.77) (width 0.6) (layer F.Cu) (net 13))
 (segment (start 108.585 65.975) (end 108.585 70.815) (width 0.6) (layer F.Cu) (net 13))
 (segment (start 107.38 64.77) (end 108.585 65.975) (width 0.6) (layer F.Cu) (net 13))
 (segment (start 106.68 59.445) (end 106.68 62.72) (width 0.6) (layer F.Cu) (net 5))
 (segment (start 109.155 57.395) (end 108.2675 58.2825) (width 0.6) (layer F.Cu) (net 5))
 (segment (start 109.855 57.395) (end 109.155 57.395) (width 0.6) (layer F.Cu) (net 5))
 (segment (start 107.38 59.445) (end 106.68 59.445) (width 0.6) (layer F.Cu) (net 5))
 (segment (start 108.2675 58.5575) (end 107.38 59.445) (width 0.6) (layer F.Cu) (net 5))
 (segment (start 108.2675 58.2825) (end 108.2675 58.5575) (width 0.6) (layer F.Cu) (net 5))
 (segment (start 103.505 64.77) (end 103.505 65.7225) (width 0.6) (layer F.Cu) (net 12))
 (segment (start 103.505 65.7225) (end 104.4575 66.675) (width 0.6) (layer F.Cu) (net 12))
 (segment (start 104.4575 66.675) (end 106.045 66.675) (width 0.6) (layer F.Cu) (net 12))
 (segment (start 107.315 67.945) (end 107.315 70.815) (width 0.6) (layer F.Cu) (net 12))
 (segment (start 106.045 66.675) (end 107.315 67.945) (width 0.6) (layer F.Cu) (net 12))
 (segment (start 103.505 59.445) (end 103.505 62.72) (width 0.6) (layer F.Cu) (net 4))
 (segment (start 105.98 57.395) (end 105.0925 58.2825) (width 0.6) (layer F.Cu) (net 4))
 (segment (start 106.68 57.395) (end 105.98 57.395) (width 0.6) (layer F.Cu) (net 4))
 (segment (start 104.205 59.445) (end 103.505 59.445) (width 0.6) (layer F.Cu) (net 4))
 (segment (start 105.0925 58.5575) (end 104.205 59.445) (width 0.6) (layer F.Cu) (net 4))
 (segment (start 105.0925 58.2825) (end 105.0925 58.5575) (width 0.6) (layer F.Cu) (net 4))
 (segment (start 100.33 64.77) (end 100.33 65.7225) (width 0.6) (layer F.Cu) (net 11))
 (segment (start 100.33 65.7225) (end 102.5525 67.945) (width 0.6) (layer F.Cu) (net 11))
 (segment (start 106.045 69.465) (end 106.045 70.815) (width 0.6) (layer F.Cu) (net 11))
 (segment (start 104.525 67.945) (end 106.045 69.465) (width 0.6) (layer F.Cu) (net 11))
 (segment (start 102.5525 67.945) (end 104.525 67.945) (width 0.6) (layer F.Cu) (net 11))
 (segment (start 100.33 59.445) (end 100.33 62.72) (width 0.6) (layer F.Cu) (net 3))
 (segment (start 102.805 57.395) (end 101.9175 58.2825) (width 0.6) (layer F.Cu) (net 3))
 (segment (start 103.505 57.395) (end 102.805 57.395) (width 0.6) (layer F.Cu) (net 3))
 (segment (start 101.03 59.445) (end 100.33 59.445) (width 0.6) (layer F.Cu) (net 3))
 (segment (start 101.9175 58.5575) (end 101.03 59.445) (width 0.6) (layer F.Cu) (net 3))
 (segment (start 101.9175 58.2825) (end 101.9175 58.5575) (width 0.6) (layer F.Cu) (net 3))
 (segment (start 104.775 69.465) (end 104.525 69.215) (width 0.6) (layer F.Cu) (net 10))
 (segment (start 104.775 70.815) (end 104.775 69.465) (width 0.6) (layer F.Cu) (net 10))
 (segment (start 104.525 69.215) (end 100.965 69.215) (width 0.6) (layer F.Cu) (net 10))
 (segment (start 97.155 65.405) (end 97.155 64.77) (width 0.6) (layer F.Cu) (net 10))
 (segment (start 100.965 69.215) (end 97.155 65.405) (width 0.6) (layer F.Cu) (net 10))
 (segment (start 97.155 59.445) (end 97.155 62.72) (width 0.6) (layer F.Cu) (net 1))
 (segment (start 99.63 57.395) (end 98.7425 58.2825) (width 0.6) (layer F.Cu) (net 1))
 (segment (start 100.33 57.395) (end 99.63 57.395) (width 0.6) (layer F.Cu) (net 1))
 (segment (start 97.855 59.445) (end 97.155 59.445) (width 0.6) (layer F.Cu) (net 1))
 (segment (start 98.7425 58.5575) (end 97.855 59.445) (width 0.6) (layer F.Cu) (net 1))
 (segment (start 98.7425 58.2825) (end 98.7425 58.5575) (width 0.6) (layer F.Cu) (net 1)))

